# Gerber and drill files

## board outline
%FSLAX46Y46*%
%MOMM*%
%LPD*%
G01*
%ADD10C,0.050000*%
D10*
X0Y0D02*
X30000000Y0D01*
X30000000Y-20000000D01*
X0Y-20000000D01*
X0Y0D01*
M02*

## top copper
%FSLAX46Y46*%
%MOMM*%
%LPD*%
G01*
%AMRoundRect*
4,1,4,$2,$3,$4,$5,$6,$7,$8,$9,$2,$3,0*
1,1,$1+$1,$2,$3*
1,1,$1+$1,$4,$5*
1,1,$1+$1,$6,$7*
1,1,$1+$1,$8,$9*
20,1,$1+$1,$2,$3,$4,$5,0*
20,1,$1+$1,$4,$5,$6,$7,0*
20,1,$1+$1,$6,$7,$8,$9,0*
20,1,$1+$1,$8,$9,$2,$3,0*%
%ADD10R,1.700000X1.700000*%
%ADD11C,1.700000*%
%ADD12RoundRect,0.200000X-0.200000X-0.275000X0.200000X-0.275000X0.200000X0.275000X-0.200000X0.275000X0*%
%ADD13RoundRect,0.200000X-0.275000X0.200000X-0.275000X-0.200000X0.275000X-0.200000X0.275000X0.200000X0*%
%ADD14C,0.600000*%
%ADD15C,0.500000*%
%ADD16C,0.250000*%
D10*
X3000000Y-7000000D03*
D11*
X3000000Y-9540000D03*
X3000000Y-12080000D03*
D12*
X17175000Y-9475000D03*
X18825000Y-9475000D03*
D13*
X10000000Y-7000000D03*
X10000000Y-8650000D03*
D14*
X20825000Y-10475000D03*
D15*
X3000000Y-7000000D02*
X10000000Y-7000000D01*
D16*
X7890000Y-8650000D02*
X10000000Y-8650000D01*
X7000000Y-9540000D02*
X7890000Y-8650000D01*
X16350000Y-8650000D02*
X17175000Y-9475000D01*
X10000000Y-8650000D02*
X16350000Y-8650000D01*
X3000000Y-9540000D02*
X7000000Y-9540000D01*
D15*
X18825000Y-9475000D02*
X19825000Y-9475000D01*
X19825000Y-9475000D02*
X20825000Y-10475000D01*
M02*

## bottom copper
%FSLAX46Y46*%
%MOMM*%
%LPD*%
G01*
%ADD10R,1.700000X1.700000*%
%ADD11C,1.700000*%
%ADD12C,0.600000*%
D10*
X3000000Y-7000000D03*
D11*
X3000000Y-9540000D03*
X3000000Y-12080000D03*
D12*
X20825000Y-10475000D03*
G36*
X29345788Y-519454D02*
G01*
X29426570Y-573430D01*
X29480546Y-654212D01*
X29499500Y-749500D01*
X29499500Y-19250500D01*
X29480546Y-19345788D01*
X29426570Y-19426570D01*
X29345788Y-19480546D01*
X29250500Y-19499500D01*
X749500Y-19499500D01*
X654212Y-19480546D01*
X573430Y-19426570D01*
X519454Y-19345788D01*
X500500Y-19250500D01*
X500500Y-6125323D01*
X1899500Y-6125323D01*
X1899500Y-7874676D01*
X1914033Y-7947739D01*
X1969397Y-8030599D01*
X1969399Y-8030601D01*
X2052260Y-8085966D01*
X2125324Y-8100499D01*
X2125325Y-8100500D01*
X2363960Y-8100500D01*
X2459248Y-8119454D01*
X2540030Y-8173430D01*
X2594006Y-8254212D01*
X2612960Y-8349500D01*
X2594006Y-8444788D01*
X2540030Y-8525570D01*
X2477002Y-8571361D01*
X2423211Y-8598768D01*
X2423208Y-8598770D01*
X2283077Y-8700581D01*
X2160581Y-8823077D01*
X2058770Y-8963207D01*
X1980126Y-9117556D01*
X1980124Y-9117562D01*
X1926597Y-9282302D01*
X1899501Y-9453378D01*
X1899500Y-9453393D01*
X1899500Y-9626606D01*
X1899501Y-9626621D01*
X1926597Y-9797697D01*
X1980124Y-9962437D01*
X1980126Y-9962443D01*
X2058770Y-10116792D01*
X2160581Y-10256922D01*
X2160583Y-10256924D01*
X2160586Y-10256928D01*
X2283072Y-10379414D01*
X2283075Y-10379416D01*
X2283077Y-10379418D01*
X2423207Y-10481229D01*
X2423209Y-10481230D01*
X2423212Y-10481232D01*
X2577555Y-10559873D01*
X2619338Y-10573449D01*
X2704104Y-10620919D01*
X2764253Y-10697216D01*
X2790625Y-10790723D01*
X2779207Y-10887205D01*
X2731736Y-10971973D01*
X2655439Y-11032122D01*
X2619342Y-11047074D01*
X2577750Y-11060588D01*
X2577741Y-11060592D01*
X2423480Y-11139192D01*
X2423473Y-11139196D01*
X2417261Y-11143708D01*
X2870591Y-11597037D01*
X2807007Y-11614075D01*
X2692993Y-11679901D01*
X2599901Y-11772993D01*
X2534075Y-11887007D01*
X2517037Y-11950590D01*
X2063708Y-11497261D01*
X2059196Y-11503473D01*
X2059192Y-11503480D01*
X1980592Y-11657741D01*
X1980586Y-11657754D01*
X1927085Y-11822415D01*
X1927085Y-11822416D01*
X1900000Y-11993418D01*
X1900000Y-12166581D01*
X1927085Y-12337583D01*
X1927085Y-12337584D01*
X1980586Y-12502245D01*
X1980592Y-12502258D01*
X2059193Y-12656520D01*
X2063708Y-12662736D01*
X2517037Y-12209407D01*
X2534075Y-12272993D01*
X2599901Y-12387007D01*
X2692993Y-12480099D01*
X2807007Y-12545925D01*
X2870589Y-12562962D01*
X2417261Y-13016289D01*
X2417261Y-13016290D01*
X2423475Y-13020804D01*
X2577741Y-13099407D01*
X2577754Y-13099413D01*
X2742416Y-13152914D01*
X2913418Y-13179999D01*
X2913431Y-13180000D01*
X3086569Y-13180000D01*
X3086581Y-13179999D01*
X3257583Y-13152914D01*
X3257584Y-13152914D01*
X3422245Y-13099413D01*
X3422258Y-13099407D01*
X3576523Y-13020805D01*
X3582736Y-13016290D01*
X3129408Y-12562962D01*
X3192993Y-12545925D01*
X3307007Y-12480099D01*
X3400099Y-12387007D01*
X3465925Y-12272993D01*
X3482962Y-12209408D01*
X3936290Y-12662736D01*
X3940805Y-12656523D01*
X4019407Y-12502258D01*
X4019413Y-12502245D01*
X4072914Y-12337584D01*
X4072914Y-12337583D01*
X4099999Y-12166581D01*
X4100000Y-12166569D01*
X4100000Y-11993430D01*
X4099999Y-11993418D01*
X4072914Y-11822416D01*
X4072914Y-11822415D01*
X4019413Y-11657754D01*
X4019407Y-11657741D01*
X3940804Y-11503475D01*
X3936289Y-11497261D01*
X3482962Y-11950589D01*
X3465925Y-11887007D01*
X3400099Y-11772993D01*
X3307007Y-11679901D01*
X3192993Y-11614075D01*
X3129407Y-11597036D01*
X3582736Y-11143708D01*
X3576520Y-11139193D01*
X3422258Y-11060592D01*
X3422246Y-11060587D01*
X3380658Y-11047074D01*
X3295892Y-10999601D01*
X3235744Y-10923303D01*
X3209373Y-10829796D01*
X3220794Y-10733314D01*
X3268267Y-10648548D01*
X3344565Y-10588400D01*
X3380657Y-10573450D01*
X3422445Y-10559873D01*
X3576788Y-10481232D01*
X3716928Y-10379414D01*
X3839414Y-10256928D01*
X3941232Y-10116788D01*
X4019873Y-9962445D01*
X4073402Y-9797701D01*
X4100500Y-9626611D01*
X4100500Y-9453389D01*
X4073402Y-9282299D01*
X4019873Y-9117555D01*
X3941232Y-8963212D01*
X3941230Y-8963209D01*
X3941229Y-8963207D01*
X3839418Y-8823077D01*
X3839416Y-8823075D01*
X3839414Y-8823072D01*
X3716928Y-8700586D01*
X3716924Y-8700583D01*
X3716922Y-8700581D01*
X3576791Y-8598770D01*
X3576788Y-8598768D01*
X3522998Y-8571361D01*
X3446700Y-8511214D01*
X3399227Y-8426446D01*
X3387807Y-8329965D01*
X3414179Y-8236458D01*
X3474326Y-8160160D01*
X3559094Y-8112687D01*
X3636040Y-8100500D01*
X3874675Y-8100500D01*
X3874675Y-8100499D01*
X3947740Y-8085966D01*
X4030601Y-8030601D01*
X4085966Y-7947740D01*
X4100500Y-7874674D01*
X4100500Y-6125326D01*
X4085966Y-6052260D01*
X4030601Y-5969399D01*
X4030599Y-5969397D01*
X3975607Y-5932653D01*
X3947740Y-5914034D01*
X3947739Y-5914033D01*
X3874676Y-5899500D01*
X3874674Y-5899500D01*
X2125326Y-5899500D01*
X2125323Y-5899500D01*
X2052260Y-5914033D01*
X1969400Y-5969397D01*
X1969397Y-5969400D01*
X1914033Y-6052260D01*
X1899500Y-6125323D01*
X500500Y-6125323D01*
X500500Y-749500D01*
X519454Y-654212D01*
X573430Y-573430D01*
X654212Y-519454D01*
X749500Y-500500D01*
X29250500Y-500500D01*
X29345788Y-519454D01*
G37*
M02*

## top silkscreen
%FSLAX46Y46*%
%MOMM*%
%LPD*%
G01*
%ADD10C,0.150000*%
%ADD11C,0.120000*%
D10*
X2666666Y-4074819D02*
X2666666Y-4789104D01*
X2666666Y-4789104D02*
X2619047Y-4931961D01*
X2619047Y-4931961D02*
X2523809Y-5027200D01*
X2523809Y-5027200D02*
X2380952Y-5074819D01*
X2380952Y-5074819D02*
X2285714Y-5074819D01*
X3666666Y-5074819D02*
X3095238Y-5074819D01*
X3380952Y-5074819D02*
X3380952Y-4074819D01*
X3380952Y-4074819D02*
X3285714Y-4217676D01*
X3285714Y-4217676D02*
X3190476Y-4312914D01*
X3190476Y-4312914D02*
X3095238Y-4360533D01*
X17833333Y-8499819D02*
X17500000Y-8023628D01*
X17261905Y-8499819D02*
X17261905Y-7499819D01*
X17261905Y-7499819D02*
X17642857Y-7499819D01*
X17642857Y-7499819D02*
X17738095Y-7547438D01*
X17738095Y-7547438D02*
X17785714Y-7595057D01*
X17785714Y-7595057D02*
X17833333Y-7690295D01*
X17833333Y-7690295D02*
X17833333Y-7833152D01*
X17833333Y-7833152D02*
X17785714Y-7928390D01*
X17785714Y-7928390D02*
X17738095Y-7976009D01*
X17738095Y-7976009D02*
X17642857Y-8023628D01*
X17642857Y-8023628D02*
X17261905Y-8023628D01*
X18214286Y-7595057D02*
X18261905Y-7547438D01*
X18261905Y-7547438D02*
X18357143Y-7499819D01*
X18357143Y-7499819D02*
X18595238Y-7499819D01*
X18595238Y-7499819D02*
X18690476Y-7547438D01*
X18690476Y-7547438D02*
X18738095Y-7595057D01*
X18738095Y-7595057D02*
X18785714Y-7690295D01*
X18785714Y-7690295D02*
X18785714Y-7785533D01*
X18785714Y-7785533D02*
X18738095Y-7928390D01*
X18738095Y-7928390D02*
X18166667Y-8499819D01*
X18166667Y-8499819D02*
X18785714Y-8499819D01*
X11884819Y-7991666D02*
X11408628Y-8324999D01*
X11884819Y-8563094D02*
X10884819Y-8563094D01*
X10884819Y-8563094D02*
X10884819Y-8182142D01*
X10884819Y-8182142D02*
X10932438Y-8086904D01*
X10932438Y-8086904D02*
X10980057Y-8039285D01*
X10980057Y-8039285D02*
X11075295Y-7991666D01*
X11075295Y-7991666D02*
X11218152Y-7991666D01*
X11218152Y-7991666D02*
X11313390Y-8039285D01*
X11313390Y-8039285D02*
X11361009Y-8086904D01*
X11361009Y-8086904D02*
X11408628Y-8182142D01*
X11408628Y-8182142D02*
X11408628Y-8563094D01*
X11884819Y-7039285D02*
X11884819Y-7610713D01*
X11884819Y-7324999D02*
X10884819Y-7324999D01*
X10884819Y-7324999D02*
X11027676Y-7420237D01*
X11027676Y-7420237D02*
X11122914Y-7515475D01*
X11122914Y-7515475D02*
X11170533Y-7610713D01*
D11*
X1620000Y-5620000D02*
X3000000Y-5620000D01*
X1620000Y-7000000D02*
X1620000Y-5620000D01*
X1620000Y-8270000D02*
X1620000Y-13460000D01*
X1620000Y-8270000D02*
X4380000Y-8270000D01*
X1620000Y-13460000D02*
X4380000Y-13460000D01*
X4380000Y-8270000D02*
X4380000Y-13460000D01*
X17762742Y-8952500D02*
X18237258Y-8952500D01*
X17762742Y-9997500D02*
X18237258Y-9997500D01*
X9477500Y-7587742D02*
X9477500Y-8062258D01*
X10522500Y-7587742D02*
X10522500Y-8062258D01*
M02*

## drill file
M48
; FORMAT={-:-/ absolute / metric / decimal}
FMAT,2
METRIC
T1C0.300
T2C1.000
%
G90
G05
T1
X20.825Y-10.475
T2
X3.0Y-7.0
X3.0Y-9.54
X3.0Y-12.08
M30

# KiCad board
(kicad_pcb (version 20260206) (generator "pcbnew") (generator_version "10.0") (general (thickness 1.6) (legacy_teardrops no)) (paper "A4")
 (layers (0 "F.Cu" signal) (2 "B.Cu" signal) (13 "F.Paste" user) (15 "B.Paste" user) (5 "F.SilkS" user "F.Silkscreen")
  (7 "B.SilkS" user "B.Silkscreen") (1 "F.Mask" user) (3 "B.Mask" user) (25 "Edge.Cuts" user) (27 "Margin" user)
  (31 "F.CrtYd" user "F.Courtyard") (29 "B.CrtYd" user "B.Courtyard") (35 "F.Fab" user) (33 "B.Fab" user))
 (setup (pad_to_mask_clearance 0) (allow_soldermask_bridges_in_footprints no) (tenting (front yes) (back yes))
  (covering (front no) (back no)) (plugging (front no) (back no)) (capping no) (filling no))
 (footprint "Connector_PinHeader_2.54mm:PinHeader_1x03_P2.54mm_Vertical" (layer "F.Cu") (at 3 7)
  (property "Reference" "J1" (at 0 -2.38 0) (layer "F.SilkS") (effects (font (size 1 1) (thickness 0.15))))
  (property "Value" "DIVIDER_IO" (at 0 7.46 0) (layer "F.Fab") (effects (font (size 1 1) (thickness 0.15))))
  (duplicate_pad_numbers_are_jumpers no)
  (fp_line (start -1.38 -1.38) (end 0 -1.38) (stroke (width 0.12) (type solid)) (layer "F.SilkS"))
  (fp_line (start -1.38 0) (end -1.38 -1.38) (stroke (width 0.12) (type solid)) (layer "F.SilkS"))
  (fp_line (start -1.38 1.27) (end -1.38 6.46) (stroke (width 0.12) (type solid)) (layer "F.SilkS"))
  (fp_line (start -1.38 1.27) (end 1.38 1.27) (stroke (width 0.12) (type solid)) (layer "F.SilkS"))
  (fp_line (start -1.38 6.46) (end 1.38 6.46) (stroke (width 0.12) (type solid)) (layer "F.SilkS"))
  (fp_line (start 1.38 1.27) (end 1.38 6.46) (stroke (width 0.12) (type solid)) (layer "F.SilkS"))
  (pad "1" thru_hole rect (at 0 0) (size 1.7 1.7) (drill 1) (layers "*.Cu" "*.Mask") (remove_unused_layers no) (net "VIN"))
  (pad "2" thru_hole circle (at 0 2.54) (size 1.7 1.7) (drill 1) (layers "*.Cu" "*.Mask") (remove_unused_layers no) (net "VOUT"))
  (pad "3" thru_hole circle (at 0 5.08) (size 1.7 1.7) (drill 1) (layers "*.Cu" "*.Mask") (remove_unused_layers no) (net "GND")))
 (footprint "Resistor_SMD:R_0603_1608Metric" (layer "F.Cu") (at 18 9.475)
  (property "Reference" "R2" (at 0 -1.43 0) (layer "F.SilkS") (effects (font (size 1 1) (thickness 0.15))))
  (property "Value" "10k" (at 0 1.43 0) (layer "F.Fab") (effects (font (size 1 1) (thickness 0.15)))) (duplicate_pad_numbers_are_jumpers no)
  (fp_line (start -0.237258 -0.5225) (end 0.237258 -0.5225) (stroke (width 0.12) (type solid)) (layer "F.SilkS"))
  (fp_line (start -0.237258 0.5225) (end 0.237258 0.5225) (stroke (width 0.12) (type solid)) (layer "F.SilkS"))
  (pad "1" smd roundrect (at -0.825 0) (size 0.8 0.95) (layers "F.Cu" "F.Mask" "F.Paste") (roundrect_rratio 0.25) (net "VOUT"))
  (pad "2" smd roundrect (at 0.825 0) (size 0.8 0.95) (layers "F.Cu" "F.Mask" "F.Paste") (roundrect_rratio 0.25) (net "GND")))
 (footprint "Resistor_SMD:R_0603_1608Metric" (layer "F.Cu") (at 10 7.825 -90)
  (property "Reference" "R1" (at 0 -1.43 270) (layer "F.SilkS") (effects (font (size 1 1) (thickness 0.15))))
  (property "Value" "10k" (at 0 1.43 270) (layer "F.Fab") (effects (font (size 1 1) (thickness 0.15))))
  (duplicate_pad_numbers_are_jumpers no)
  (fp_line (start -0.237258 0.5225) (end 0.237258 0.5225) (stroke (width 0.12) (type solid)) (layer "F.SilkS"))
  (fp_line (start -0.237258 -0.5225) (end 0.237258 -0.5225) (stroke (width 0.12) (type solid)) (layer "F.SilkS"))
  (pad "1" smd roundrect (at -0.825 0 270) (size 0.8 0.95) (layers "F.Cu" "F.Mask" "F.Paste") (roundrect_rratio 0.25) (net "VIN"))
  (pad "2" smd roundrect (at 0.825 0 270) (size 0.8 0.95) (layers "F.Cu" "F.Mask" "F.Paste") (roundrect_rratio 0.25) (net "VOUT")))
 (gr_rect (start 0 0) (end 30 20) (stroke (width 0.05) (type default)) (fill no) (layer "Edge.Cuts"))
 (segment (start 3 7) (end 10 7) (width 0.5) (layer "F.Cu") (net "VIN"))
 (segment (start 7.89 8.65) (end 10 8.65) (width 0.25) (layer "F.Cu") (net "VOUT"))
 (segment (start 7 9.54) (end 7.89 8.65) (width 0.25) (layer "F.Cu") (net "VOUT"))
 (segment (start 16.35 8.65) (end 17.175 9.475) (width 0.25) (layer "F.Cu") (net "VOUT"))
 (segment (start 10 8.65) (end 16.35 8.65) (width 0.25) (layer "F.Cu") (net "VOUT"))
 (segment (start 3 9.54) (end 7 9.54) (width 0.25) (layer "F.Cu") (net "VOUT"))
 (segment (start 18.825 9.475) (end 19.825 9.475) (width 0.5) (layer "F.Cu") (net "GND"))
 (segment (start 19.825 9.475) (end 20.825 10.475) (width 0.5) (layer "F.Cu") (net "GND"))
 (via (at 20.825 10.475) (size 0.6) (drill 0.3) (layers "F.Cu" "B.Cu") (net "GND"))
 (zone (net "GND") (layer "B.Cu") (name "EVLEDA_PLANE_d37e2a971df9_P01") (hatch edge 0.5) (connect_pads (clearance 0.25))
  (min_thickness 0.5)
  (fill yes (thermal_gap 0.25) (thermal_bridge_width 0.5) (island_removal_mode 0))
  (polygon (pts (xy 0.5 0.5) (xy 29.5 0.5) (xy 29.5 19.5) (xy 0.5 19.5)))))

